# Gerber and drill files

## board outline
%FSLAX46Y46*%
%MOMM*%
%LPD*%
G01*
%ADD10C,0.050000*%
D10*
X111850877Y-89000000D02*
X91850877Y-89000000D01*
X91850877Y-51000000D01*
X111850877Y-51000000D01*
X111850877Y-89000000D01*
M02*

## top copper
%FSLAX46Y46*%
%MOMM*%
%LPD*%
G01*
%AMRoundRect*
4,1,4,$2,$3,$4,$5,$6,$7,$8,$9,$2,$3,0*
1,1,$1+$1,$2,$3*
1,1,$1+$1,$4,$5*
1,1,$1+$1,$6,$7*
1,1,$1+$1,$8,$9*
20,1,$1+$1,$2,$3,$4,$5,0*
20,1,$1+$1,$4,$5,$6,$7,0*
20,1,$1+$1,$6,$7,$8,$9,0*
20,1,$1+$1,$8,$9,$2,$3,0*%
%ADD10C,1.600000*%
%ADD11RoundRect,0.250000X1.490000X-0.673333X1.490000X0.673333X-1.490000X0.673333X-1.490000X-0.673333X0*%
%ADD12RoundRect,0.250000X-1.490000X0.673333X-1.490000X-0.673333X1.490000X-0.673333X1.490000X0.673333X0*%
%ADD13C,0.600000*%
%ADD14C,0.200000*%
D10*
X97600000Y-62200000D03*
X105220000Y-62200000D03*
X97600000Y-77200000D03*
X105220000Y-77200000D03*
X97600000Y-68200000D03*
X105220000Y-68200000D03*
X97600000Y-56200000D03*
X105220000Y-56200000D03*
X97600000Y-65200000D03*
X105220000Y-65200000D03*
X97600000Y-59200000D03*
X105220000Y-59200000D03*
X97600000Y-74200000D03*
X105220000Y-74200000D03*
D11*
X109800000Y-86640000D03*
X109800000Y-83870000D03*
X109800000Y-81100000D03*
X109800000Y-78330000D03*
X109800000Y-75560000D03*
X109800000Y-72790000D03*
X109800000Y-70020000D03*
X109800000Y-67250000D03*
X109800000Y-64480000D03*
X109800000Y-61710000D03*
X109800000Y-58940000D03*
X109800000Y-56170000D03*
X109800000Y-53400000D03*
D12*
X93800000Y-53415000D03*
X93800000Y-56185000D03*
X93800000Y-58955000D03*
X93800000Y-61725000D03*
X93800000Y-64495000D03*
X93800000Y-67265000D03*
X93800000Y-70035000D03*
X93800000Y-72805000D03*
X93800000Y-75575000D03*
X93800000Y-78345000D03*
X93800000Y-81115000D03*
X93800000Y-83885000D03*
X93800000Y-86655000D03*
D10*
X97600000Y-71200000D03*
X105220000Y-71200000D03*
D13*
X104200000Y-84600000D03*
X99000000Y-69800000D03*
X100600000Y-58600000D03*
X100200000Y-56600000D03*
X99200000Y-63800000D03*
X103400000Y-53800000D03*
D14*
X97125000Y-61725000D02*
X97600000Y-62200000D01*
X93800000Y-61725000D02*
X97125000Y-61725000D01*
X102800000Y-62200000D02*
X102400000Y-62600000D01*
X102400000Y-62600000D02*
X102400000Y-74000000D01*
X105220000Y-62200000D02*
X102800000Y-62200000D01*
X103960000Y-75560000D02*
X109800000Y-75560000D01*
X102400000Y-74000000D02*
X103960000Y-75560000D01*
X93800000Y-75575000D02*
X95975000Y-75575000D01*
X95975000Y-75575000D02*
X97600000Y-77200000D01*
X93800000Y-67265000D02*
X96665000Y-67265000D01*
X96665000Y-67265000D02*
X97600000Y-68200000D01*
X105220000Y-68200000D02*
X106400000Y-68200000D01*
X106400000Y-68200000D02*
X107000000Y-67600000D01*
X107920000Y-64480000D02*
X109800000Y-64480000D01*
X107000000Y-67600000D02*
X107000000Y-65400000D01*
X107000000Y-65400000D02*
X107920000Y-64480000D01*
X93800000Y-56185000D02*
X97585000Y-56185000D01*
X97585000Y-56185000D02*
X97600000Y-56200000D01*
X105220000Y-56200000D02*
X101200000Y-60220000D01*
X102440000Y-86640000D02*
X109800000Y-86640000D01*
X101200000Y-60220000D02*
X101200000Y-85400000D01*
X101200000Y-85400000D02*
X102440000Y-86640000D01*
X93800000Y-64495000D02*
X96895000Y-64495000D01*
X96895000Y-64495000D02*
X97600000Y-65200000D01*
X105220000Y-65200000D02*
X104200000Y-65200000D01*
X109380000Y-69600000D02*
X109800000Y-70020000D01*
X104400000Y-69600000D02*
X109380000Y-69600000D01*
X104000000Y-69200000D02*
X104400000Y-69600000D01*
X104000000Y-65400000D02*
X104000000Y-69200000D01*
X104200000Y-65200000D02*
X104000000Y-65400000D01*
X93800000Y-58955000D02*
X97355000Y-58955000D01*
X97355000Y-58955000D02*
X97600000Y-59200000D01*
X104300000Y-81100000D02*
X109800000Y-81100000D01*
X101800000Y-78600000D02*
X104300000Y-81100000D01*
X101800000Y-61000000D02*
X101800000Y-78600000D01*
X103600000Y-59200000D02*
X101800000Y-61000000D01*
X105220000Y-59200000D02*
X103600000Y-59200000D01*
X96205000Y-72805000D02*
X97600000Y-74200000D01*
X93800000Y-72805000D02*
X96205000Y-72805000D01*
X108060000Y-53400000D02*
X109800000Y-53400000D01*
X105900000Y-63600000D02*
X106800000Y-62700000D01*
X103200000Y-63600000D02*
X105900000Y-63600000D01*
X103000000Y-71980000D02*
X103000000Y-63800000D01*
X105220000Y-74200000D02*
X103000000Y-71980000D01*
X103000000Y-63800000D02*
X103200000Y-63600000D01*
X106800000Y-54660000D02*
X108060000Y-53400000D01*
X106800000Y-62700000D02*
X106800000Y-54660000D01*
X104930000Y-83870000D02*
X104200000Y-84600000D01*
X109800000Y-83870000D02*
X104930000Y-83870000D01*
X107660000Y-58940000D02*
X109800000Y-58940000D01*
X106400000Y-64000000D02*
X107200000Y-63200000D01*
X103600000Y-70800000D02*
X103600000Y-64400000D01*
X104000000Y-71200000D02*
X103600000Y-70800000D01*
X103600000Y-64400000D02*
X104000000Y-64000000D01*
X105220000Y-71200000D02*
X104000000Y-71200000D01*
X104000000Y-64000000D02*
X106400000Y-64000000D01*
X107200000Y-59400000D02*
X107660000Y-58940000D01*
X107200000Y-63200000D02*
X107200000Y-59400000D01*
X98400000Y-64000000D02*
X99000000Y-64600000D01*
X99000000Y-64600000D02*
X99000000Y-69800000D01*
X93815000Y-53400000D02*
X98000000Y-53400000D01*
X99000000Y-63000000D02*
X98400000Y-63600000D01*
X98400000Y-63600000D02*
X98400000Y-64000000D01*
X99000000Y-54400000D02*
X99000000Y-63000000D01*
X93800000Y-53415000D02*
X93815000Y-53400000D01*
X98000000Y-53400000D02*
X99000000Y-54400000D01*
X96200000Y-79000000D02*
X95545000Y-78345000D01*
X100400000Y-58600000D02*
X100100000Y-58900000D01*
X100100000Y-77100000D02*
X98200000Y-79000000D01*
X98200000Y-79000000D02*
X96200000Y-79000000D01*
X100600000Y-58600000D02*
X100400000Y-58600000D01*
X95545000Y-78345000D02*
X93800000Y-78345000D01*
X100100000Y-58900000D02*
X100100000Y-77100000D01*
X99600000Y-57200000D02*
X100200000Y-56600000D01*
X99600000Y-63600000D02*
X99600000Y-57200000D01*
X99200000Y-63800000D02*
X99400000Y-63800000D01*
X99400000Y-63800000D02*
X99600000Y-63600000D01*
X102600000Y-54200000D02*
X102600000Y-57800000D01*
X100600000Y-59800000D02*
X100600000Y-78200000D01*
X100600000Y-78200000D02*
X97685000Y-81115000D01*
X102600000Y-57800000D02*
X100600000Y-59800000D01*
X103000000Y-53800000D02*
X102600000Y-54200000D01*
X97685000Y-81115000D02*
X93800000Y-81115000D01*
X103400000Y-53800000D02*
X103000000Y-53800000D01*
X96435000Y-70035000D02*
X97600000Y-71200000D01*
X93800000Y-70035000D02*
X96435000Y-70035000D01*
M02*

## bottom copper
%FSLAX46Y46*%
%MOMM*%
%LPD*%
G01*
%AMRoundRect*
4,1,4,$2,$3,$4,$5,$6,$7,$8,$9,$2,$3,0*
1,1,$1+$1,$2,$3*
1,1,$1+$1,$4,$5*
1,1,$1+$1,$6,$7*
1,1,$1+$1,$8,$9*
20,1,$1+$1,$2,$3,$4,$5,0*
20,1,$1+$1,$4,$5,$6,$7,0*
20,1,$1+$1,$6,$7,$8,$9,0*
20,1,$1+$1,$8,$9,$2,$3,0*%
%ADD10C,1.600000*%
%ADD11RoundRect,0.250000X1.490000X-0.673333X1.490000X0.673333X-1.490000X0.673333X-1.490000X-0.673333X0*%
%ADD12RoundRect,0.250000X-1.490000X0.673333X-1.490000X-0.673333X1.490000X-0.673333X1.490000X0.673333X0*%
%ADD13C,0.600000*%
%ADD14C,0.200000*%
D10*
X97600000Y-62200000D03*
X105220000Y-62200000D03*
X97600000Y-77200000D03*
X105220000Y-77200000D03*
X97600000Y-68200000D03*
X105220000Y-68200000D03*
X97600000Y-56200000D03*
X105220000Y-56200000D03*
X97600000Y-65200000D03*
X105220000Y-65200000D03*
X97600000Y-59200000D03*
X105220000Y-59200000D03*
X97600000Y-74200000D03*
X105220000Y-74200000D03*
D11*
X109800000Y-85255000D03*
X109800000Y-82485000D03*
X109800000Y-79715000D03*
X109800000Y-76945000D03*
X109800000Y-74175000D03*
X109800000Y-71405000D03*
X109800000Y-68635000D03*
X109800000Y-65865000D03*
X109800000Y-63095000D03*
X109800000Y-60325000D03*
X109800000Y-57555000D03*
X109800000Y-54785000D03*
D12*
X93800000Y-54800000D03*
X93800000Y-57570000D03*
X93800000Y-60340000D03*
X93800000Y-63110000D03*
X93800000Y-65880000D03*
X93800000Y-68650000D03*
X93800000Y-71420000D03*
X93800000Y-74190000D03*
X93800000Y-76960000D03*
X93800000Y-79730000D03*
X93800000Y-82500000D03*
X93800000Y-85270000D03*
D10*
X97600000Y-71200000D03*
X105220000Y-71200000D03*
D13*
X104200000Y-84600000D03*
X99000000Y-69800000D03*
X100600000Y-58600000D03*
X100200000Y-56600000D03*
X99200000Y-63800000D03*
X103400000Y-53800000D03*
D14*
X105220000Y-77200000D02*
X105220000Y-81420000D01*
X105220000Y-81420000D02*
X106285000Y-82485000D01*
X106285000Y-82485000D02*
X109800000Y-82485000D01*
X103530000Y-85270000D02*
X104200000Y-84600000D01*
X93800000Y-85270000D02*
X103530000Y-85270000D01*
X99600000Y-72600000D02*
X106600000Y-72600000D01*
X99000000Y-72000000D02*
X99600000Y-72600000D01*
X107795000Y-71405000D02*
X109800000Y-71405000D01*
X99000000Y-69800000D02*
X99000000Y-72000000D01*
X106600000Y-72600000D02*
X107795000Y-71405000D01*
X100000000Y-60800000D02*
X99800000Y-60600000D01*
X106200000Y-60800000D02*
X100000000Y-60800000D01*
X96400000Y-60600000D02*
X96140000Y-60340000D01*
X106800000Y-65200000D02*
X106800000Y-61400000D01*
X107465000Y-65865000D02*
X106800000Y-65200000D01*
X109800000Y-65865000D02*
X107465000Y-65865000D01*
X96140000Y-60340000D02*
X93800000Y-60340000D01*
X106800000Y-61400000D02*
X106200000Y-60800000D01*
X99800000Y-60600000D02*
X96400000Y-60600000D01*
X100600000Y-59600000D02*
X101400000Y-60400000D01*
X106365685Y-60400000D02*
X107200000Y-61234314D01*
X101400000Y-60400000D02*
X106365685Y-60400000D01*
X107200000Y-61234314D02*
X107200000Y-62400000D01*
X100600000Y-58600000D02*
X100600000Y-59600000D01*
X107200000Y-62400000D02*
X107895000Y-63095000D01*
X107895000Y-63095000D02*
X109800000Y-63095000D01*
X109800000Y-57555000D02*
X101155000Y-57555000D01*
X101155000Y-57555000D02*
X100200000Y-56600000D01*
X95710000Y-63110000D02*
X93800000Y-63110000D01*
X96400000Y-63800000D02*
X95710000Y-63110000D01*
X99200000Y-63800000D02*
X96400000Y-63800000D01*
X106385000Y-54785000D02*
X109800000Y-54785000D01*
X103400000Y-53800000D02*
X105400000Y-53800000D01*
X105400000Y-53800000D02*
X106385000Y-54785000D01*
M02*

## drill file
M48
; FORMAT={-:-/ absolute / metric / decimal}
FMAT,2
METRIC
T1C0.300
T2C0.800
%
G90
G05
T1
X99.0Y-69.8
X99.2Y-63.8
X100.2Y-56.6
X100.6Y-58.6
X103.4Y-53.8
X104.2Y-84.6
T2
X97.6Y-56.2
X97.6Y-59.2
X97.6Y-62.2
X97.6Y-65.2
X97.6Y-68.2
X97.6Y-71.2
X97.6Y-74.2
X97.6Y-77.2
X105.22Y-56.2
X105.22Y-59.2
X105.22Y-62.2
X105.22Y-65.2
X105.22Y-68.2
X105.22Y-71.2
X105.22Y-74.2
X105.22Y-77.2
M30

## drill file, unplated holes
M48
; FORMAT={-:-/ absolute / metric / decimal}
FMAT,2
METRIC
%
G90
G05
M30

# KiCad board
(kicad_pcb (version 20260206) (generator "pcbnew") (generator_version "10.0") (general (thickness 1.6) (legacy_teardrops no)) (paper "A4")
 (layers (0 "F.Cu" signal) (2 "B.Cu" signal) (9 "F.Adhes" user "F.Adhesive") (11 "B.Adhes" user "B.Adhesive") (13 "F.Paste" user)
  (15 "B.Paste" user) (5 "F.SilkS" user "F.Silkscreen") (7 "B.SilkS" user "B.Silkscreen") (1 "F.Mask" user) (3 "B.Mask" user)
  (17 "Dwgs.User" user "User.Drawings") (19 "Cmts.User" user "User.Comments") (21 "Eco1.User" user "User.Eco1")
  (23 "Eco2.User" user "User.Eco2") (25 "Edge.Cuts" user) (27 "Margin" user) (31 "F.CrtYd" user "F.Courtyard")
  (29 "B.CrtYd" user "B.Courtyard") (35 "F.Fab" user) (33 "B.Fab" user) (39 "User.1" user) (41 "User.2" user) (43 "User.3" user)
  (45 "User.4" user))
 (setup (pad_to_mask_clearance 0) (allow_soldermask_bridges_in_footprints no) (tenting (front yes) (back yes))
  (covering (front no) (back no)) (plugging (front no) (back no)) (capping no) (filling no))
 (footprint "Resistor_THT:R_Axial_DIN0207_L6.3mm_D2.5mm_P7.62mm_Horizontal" (layer "F.Cu") (at 97.6 62.2)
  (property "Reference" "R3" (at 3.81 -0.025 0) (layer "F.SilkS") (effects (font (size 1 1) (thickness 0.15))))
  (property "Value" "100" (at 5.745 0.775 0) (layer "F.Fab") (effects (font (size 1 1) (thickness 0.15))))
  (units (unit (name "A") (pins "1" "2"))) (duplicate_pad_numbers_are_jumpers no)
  (pad "1" thru_hole circle (at 0 0) (size 1.6 1.6) (drill 0.8) (layers "*.Cu" "*.Mask") (remove_unused_layers no) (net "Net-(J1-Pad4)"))
  (pad "2" thru_hole circle (at 7.62 0) (size 1.6 1.6) (drill 0.8) (layers "*.Cu" "*.Mask") (remove_unused_layers no) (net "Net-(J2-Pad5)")))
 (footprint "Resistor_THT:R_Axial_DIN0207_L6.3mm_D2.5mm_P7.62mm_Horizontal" (layer "F.Cu") (at 97.6 77.2)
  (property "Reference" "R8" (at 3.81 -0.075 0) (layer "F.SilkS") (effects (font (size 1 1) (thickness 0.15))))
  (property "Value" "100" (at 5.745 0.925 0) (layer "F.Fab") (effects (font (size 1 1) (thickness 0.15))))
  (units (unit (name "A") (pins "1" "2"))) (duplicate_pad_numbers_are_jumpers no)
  (pad "1" thru_hole circle (at 0 0) (size 1.6 1.6) (drill 0.8) (layers "*.Cu" "*.Mask") (remove_unused_layers no) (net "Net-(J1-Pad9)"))
  (pad "2" thru_hole circle (at 7.62 0) (size 1.6 1.6) (drill 0.8) (layers "*.Cu" "*.Mask") (remove_unused_layers no) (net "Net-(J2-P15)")))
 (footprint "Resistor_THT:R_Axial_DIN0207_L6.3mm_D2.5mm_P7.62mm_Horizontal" (layer "F.Cu") (at 97.6 68.2)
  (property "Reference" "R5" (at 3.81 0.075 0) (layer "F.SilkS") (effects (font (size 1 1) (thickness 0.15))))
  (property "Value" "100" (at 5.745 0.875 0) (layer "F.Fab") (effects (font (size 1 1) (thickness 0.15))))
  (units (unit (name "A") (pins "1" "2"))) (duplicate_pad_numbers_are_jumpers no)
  (pad "1" thru_hole circle (at 0 0) (size 1.6 1.6) (drill 0.8) (layers "*.Cu" "*.Mask") (remove_unused_layers no) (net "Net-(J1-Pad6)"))
  (pad "2" thru_hole circle (at 7.62 0) (size 1.6 1.6) (drill 0.8) (layers "*.Cu" "*.Mask") (remove_unused_layers no) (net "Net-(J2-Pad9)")))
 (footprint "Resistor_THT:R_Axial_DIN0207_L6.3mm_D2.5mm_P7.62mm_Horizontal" (layer "F.Cu") (at 97.6 56.2)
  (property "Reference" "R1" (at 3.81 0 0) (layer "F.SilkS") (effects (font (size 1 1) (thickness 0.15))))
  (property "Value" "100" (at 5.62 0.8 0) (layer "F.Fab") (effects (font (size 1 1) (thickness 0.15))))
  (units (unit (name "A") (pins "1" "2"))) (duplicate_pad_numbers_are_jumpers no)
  (pad "1" thru_hole circle (at 0 0) (size 1.6 1.6) (drill 0.8) (layers "*.Cu" "*.Mask") (remove_unused_layers no) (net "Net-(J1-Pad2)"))
  (pad "2" thru_hole circle (at 7.62 0) (size 1.6 1.6) (drill 0.8) (layers "*.Cu" "*.Mask") (remove_unused_layers no) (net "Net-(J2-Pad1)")))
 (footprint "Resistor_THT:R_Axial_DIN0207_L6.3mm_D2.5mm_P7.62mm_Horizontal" (layer "F.Cu") (at 97.6 65.2)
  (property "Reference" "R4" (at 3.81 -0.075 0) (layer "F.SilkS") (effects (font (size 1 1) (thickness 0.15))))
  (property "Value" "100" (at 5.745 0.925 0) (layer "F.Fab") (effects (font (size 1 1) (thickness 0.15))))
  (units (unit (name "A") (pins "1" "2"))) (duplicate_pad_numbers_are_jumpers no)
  (pad "1" thru_hole circle (at 0 0) (size 1.6 1.6) (drill 0.8) (layers "*.Cu" "*.Mask") (remove_unused_layers no) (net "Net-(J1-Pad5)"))
  (pad "2" thru_hole circle (at 7.62 0) (size 1.6 1.6) (drill 0.8) (layers "*.Cu" "*.Mask") (remove_unused_layers no) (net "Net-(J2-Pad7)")))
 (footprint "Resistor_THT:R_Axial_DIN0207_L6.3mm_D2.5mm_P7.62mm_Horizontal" (layer "F.Cu") (at 97.6 59.2)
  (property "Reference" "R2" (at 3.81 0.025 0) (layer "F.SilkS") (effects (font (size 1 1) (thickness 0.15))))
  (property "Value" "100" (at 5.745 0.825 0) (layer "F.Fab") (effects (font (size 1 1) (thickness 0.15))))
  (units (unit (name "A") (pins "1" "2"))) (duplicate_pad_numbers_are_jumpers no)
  (pad "1" thru_hole circle (at 0 0) (size 1.6 1.6) (drill 0.8) (layers "*.Cu" "*.Mask") (remove_unused_layers no) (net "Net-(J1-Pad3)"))
  (pad "2" thru_hole circle (at 7.62 0) (size 1.6 1.6) (drill 0.8) (layers "*.Cu" "*.Mask") (remove_unused_layers no) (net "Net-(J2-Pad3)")))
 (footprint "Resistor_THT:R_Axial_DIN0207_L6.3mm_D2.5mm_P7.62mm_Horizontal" (layer "F.Cu") (at 97.6 74.2)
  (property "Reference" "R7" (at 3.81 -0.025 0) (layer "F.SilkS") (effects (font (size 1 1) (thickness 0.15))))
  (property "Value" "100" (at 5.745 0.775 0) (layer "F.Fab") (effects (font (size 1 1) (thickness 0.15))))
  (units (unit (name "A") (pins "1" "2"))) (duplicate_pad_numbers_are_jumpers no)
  (pad "1" thru_hole circle (at 0 0) (size 1.6 1.6) (drill 0.8) (layers "*.Cu" "*.Mask") (remove_unused_layers no) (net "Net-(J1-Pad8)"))
  (pad "2" thru_hole circle (at 7.62 0) (size 1.6 1.6) (drill 0.8) (layers "*.Cu" "*.Mask") (remove_unused_layers no) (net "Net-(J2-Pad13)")))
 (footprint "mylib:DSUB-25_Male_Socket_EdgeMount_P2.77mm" (layer "F.Cu") (at 116.84 77.06 180)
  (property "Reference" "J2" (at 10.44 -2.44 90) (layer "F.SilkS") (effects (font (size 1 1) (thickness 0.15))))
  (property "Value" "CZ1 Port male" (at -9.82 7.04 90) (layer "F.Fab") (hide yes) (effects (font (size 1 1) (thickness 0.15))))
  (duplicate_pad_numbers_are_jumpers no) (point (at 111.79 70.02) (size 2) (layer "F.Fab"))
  (pad "1" smd roundrect (at 7.04 -9.58 90) (size 1.846667 3.48) (layers "F.Cu" "F.Mask" "F.Paste") (roundrect_rratio 0.135379)
   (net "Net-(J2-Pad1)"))
  (pad "2" smd roundrect (at 7.04 -6.81 90) (size 1.846667 3.48) (layers "F.Cu" "F.Mask" "F.Paste") (roundrect_rratio 0.135379) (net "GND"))
  (pad "3" smd roundrect (at 7.04 -4.04 90) (size 1.846667 3.48) (layers "F.Cu" "F.Mask" "F.Paste") (roundrect_rratio 0.135379)
   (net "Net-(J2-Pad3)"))
  (pad "4" smd roundrect (at 7.04 -1.27 90) (size 1.846667 3.48) (layers "F.Cu" "F.Mask" "F.Paste") (roundrect_rratio 0.135379)
   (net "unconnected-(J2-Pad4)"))
  (pad "5" smd roundrect (at 7.04 1.5 90) (size 1.846667 3.48) (layers "F.Cu" "F.Mask" "F.Paste") (roundrect_rratio 0.135379)
   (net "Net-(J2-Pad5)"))
  (pad "6" smd roundrect (at 7.04 4.27 90) (size 1.846667 3.48) (layers "F.Cu" "F.Mask" "F.Paste") (roundrect_rratio 0.135379)
   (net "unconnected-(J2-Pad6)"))
  (pad "7" smd roundrect (at 7.04 7.04 90) (size 1.846667 3.48) (layers "F.Cu" "F.Mask" "F.Paste") (roundrect_rratio 0.135379)
   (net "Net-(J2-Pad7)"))
  (pad "8" smd roundrect (at 7.04 9.81 90) (size 1.846667 3.48) (layers "F.Cu" "F.Mask" "F.Paste") (roundrect_rratio 0.135379)
   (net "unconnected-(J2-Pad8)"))
  (pad "9" smd roundrect (at 7.04 12.58 90) (size 1.846667 3.48) (layers "F.Cu" "F.Mask" "F.Paste") (roundrect_rratio 0.135379)
   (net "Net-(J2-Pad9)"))
  (pad "10" smd roundrect (at 7.04 15.35 90) (size 1.846667 3.48) (layers "F.Cu" "F.Mask" "F.Paste") (roundrect_rratio 0.135379)
   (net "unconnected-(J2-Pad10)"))
  (pad "11" smd roundrect (at 7.04 18.12 90) (size 1.846667 3.48) (layers "F.Cu" "F.Mask" "F.Paste") (roundrect_rratio 0.135379)
   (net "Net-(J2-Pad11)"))
  (pad "12" smd roundrect (at 7.04 20.89 90) (size 1.846667 3.48) (layers "F.Cu" "F.Mask" "F.Paste") (roundrect_rratio 0.135379)
   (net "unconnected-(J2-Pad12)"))
  (pad "13" smd roundrect (at 7.04 23.66 90) (size 1.846667 3.48) (layers "F.Cu" "F.Mask" "F.Paste") (roundrect_rratio 0.135379)
   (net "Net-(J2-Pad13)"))
  (pad "14" smd roundrect (at 7.04 -8.195 90) (size 1.846667 3.48) (layers "B.Cu" "B.Mask" "B.Paste") (roundrect_rratio 0.135379)
   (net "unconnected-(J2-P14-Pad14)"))
  (pad "15" smd roundrect (at 7.04 -5.425 90) (size 1.846667 3.48) (layers "B.Cu" "B.Mask" "B.Paste") (roundrect_rratio 0.135379)
   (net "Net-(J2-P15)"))
  (pad "16" smd roundrect (at 7.04 -2.655 90) (size 1.846667 3.48) (layers "B.Cu" "B.Mask" "B.Paste") (roundrect_rratio 0.135379)
   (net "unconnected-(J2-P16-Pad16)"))
  (pad "17" smd roundrect (at 7.04 0.115 90) (size 1.846667 3.48) (layers "B.Cu" "B.Mask" "B.Paste") (roundrect_rratio 0.135379)
   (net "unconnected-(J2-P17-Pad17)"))
  (pad "18" smd roundrect (at 7.04 2.885 90) (size 1.846667 3.48) (layers "B.Cu" "B.Mask" "B.Paste") (roundrect_rratio 0.135379)
   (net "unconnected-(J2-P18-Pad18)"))
  (pad "19" smd roundrect (at 7.04 5.655 90) (size 1.846667 3.48) (layers "B.Cu" "B.Mask" "B.Paste") (roundrect_rratio 0.135379)
   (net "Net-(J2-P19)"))
  (pad "20" smd roundrect (at 7.04 8.425 90) (size 1.846667 3.48) (layers "B.Cu" "B.Mask" "B.Paste") (roundrect_rratio 0.135379)
   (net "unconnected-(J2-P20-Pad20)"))
  (pad "21" smd roundrect (at 7.04 11.195 90) (size 1.846667 3.48) (layers "B.Cu" "B.Mask" "B.Paste") (roundrect_rratio 0.135379)
   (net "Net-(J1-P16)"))
  (pad "22" smd roundrect (at 7.04 13.965 90) (size 1.846667 3.48) (layers "B.Cu" "B.Mask" "B.Paste") (roundrect_rratio 0.135379)
   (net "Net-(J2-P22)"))
  (pad "23" smd roundrect (at 7.04 16.735 90) (size 1.846667 3.48) (layers "B.Cu" "B.Mask" "B.Paste") (roundrect_rratio 0.135379)
   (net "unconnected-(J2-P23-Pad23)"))
  (pad "24" smd roundrect (at 7.04 19.505 90) (size 1.846667 3.48) (layers "B.Cu" "B.Mask" "B.Paste") (roundrect_rratio 0.135379)
   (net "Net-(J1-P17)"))
  (pad "25" smd roundrect (at 7.04 22.275 90) (size 1.846667 3.48) (layers "B.Cu" "B.Mask" "B.Paste") (roundrect_rratio 0.135379)
   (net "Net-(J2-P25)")))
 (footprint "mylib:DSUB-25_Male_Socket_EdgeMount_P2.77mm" (layer "F.Cu") (at 86.76 62.995)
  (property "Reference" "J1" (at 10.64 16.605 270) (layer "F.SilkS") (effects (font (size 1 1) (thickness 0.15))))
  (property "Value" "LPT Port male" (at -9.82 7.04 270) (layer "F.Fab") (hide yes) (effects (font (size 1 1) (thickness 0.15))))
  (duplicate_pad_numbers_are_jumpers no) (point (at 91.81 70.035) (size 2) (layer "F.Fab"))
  (pad "1" smd roundrect (at 7.04 -9.58 270) (size 1.846667 3.48) (layers "F.Cu" "F.Mask" "F.Paste") (roundrect_rratio 0.135379)
   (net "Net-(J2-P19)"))
  (pad "2" smd roundrect (at 7.04 -6.81 270) (size 1.846667 3.48) (layers "F.Cu" "F.Mask" "F.Paste") (roundrect_rratio 0.135379)
   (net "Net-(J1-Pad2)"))
  (pad "3" smd roundrect (at 7.04 -4.04 270) (size 1.846667 3.48) (layers "F.Cu" "F.Mask" "F.Paste") (roundrect_rratio 0.135379)
   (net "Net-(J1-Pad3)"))
  (pad "4" smd roundrect (at 7.04 -1.27 270) (size 1.846667 3.48) (layers "F.Cu" "F.Mask" "F.Paste") (roundrect_rratio 0.135379)
   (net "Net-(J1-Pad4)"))
  (pad "5" smd roundrect (at 7.04 1.5 270) (size 1.846667 3.48) (layers "F.Cu" "F.Mask" "F.Paste") (roundrect_rratio 0.135379)
   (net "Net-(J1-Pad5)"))
  (pad "6" smd roundrect (at 7.04 4.27 270) (size 1.846667 3.48) (layers "F.Cu" "F.Mask" "F.Paste") (roundrect_rratio 0.135379)
   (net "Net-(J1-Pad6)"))
  (pad "7" smd roundrect (at 7.04 7.04 270) (size 1.846667 3.48) (layers "F.Cu" "F.Mask" "F.Paste") (roundrect_rratio 0.135379)
   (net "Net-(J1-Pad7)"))
  (pad "8" smd roundrect (at 7.04 9.81 270) (size 1.846667 3.48) (layers "F.Cu" "F.Mask" "F.Paste") (roundrect_rratio 0.135379)
   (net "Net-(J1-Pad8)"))
  (pad "9" smd roundrect (at 7.04 12.58 270) (size 1.846667 3.48) (layers "F.Cu" "F.Mask" "F.Paste") (roundrect_rratio 0.135379)
   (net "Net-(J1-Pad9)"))
  (pad "10" smd roundrect (at 7.04 15.35 270) (size 1.846667 3.48) (layers "F.Cu" "F.Mask" "F.Paste") (roundrect_rratio 0.135379)
   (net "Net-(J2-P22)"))
  (pad "11" smd roundrect (at 7.04 18.12 270) (size 1.846667 3.48) (layers "F.Cu" "F.Mask" "F.Paste") (roundrect_rratio 0.135379)
   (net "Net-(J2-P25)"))
  (pad "12" smd roundrect (at 7.04 20.89 270) (size 1.846667 3.48) (layers "F.Cu" "F.Mask" "F.Paste") (roundrect_rratio 0.135379)
   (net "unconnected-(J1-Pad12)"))
  (pad "13" smd roundrect (at 7.04 23.66 270) (size 1.846667 3.48) (layers "F.Cu" "F.Mask" "F.Paste") (roundrect_rratio 0.135379)
   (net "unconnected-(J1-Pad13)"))
  (pad "14" smd roundrect (at 7.04 -8.195 270) (size 1.846667 3.48) (layers "B.Cu" "B.Mask" "B.Paste") (roundrect_rratio 0.135379)
   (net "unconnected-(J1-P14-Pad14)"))
  (pad "15" smd roundrect (at 7.04 -5.425 270) (size 1.846667 3.48) (layers "B.Cu" "B.Mask" "B.Paste") (roundrect_rratio 0.135379)
   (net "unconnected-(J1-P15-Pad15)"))
  (pad "16" smd roundrect (at 7.04 -2.655 270) (size 1.846667 3.48) (layers "B.Cu" "B.Mask" "B.Paste") (roundrect_rratio 0.135379)
   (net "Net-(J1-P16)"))
  (pad "17" smd roundrect (at 7.04 0.115 270) (size 1.846667 3.48) (layers "B.Cu" "B.Mask" "B.Paste") (roundrect_rratio 0.135379)
   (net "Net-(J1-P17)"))
  (pad "18" smd roundrect (at 7.04 2.885 270) (size 1.846667 3.48) (layers "B.Cu" "B.Mask" "B.Paste") (roundrect_rratio 0.135379)
   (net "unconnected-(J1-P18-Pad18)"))
  (pad "19" smd roundrect (at 7.04 5.655 270) (size 1.846667 3.48) (layers "B.Cu" "B.Mask" "B.Paste") (roundrect_rratio 0.135379)
   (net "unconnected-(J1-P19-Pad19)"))
  (pad "20" smd roundrect (at 7.04 8.425 270) (size 1.846667 3.48) (layers "B.Cu" "B.Mask" "B.Paste") (roundrect_rratio 0.135379)
   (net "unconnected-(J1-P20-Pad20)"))
  (pad "21" smd roundrect (at 7.04 11.195 270) (size 1.846667 3.48) (layers "B.Cu" "B.Mask" "B.Paste") (roundrect_rratio 0.135379)
   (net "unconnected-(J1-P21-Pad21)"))
  (pad "22" smd roundrect (at 7.04 13.965 270) (size 1.846667 3.48) (layers "B.Cu" "B.Mask" "B.Paste") (roundrect_rratio 0.135379)
   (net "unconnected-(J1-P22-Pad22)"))
  (pad "23" smd roundrect (at 7.04 16.735 270) (size 1.846667 3.48) (layers "B.Cu" "B.Mask" "B.Paste") (roundrect_rratio 0.135379)
   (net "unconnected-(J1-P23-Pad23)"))
  (pad "24" smd roundrect (at 7.04 19.505 270) (size 1.846667 3.48) (layers "B.Cu" "B.Mask" "B.Paste") (roundrect_rratio 0.135379)
   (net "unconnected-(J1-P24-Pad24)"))
  (pad "25" smd roundrect (at 7.04 22.275 270) (size 1.846667 3.48) (layers "B.Cu" "B.Mask" "B.Paste") (roundrect_rratio 0.135379)
   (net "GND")))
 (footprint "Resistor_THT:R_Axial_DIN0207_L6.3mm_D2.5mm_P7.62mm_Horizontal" (layer "F.Cu") (at 97.6 71.2)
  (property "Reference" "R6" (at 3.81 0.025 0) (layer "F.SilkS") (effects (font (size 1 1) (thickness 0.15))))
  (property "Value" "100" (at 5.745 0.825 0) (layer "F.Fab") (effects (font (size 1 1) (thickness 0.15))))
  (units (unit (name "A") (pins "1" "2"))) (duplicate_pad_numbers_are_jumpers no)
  (pad "1" thru_hole circle (at 0 0) (size 1.6 1.6) (drill 0.8) (layers "*.Cu" "*.Mask") (remove_unused_layers no) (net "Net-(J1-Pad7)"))
  (pad "2" thru_hole circle (at 7.62 0) (size 1.6 1.6) (drill 0.8) (layers "*.Cu" "*.Mask") (remove_unused_layers no) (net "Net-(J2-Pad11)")))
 (gr_poly
  (pts (xy 91.850877 51) (xy 91.850877 89) (xy 111.850877 89) (xy 111.850877 51)) (stroke (width 0.05) (type solid)) (fill no)
  (layer "Edge.Cuts"))
 (segment (start 97.125 61.725) (end 97.6 62.2) (width 0.2) (layer "F.Cu") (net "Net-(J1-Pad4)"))
 (segment (start 93.8 61.725) (end 97.125 61.725) (width 0.2) (layer "F.Cu") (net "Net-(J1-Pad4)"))
 (segment (start 102.8 62.2) (end 102.4 62.6) (width 0.2) (layer "F.Cu") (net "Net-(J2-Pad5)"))
 (segment (start 102.4 62.6) (end 102.4 74) (width 0.2) (layer "F.Cu") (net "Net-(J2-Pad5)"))
 (segment (start 105.22 62.2) (end 102.8 62.2) (width 0.2) (layer "F.Cu") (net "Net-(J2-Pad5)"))
 (segment (start 103.96 75.56) (end 109.8 75.56) (width 0.2) (layer "F.Cu") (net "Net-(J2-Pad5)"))
 (segment (start 102.4 74) (end 103.96 75.56) (width 0.2) (layer "F.Cu") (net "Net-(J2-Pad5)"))
 (segment (start 93.8 75.575) (end 95.975 75.575) (width 0.2) (layer "F.Cu") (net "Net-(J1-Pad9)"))
 (segment (start 95.975 75.575) (end 97.6 77.2) (width 0.2) (layer "F.Cu") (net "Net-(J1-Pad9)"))
 (segment (start 105.22 77.2) (end 105.22 81.42) (width 0.2) (layer "B.Cu") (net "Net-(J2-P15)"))
 (segment (start 105.22 81.42) (end 106.285 82.485) (width 0.2) (layer "B.Cu") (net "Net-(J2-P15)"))
 (segment (start 106.285 82.485) (end 109.8 82.485) (width 0.2) (layer "B.Cu") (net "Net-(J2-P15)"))
 (segment (start 93.8 67.265) (end 96.665 67.265) (width 0.2) (layer "F.Cu") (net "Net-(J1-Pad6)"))
 (segment (start 96.665 67.265) (end 97.6 68.2) (width 0.2) (layer "F.Cu") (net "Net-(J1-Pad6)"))
 (segment (start 105.22 68.2) (end 106.4 68.2) (width 0.2) (layer "F.Cu") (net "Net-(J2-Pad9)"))
 (segment (start 106.4 68.2) (end 107 67.6) (width 0.2) (layer "F.Cu") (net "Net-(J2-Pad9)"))
 (segment (start 107.92 64.48) (end 109.8 64.48) (width 0.2) (layer "F.Cu") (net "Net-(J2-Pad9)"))
 (segment (start 107 67.6) (end 107 65.4) (width 0.2) (layer "F.Cu") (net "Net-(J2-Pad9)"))
 (segment (start 107 65.4) (end 107.92 64.48) (width 0.2) (layer "F.Cu") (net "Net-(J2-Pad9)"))
 (segment (start 93.8 56.185) (end 97.585 56.185) (width 0.2) (layer "F.Cu") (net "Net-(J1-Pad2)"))
 (segment (start 97.585 56.185) (end 97.6 56.2) (width 0.2) (layer "F.Cu") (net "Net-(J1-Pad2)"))
 (segment (start 105.22 56.2) (end 101.2 60.22) (width 0.2) (layer "F.Cu") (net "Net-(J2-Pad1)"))
 (segment (start 102.44 86.64) (end 109.8 86.64) (width 0.2) (layer "F.Cu") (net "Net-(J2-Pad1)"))
 (segment (start 101.2 60.22) (end 101.2 85.4) (width 0.2) (layer "F.Cu") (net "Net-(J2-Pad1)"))
 (segment (start 101.2 85.4) (end 102.44 86.64) (width 0.2) (layer "F.Cu") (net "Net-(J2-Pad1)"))
 (segment (start 93.8 64.495) (end 96.895 64.495) (width 0.2) (layer "F.Cu") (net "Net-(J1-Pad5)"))
 (segment (start 96.895 64.495) (end 97.6 65.2) (width 0.2) (layer "F.Cu") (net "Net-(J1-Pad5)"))
 (segment (start 105.22 65.2) (end 104.2 65.2) (width 0.2) (layer "F.Cu") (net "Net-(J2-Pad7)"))
 (segment (start 109.38 69.6) (end 109.8 70.02) (width 0.2) (layer "F.Cu") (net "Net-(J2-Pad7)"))
 (segment (start 104.4 69.6) (end 109.38 69.6) (width 0.2) (layer "F.Cu") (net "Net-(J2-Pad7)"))
 (segment (start 104 69.2) (end 104.4 69.6) (width 0.2) (layer "F.Cu") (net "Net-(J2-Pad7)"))
 (segment (start 104 65.4) (end 104 69.2) (width 0.2) (layer "F.Cu") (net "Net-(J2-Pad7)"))
 (segment (start 104.2 65.2) (end 104 65.4) (width 0.2) (layer "F.Cu") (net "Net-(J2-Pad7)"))
 (segment (start 93.8 58.955) (end 97.355 58.955) (width 0.2) (layer "F.Cu") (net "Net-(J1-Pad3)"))
 (segment (start 97.355 58.955) (end 97.6 59.2) (width 0.2) (layer "F.Cu") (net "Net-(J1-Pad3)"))
 (segment (start 104.3 81.1) (end 109.8 81.1) (width 0.2) (layer "F.Cu") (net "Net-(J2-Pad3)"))
 (segment (start 101.8 78.6) (end 104.3 81.1) (width 0.2) (layer "F.Cu") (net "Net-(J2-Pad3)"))
 (segment (start 101.8 61) (end 101.8 78.6) (width 0.2) (layer "F.Cu") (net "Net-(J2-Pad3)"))
 (segment (start 103.6 59.2) (end 101.8 61) (width 0.2) (layer "F.Cu") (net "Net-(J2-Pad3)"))
 (segment (start 105.22 59.2) (end 103.6 59.2) (width 0.2) (layer "F.Cu") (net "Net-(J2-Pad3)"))
 (segment (start 96.205 72.805) (end 97.6 74.2) (width 0.2) (layer "F.Cu") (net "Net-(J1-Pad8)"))
 (segment (start 93.8 72.805) (end 96.205 72.805) (width 0.2) (layer "F.Cu") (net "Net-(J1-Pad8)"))
 (segment (start 108.06 53.4) (end 109.8 53.4) (width 0.2) (layer "F.Cu") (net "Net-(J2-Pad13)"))
 (segment (start 105.9 63.6) (end 106.8 62.7) (width 0.2) (layer "F.Cu") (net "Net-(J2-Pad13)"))
 (segment (start 103.2 63.6) (end 105.9 63.6) (width 0.2) (layer "F.Cu") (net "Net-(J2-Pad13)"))
 (segment (start 103 71.98) (end 103 63.8) (width 0.2) (layer "F.Cu") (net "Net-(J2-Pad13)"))
 (segment (start 105.22 74.2) (end 103 71.98) (width 0.2) (layer "F.Cu") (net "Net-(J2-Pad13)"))
 (segment (start 103 63.8) (end 103.2 63.6) (width 0.2) (layer "F.Cu") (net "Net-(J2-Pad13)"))
 (segment (start 106.8 54.66) (end 108.06 53.4) (width 0.2) (layer "F.Cu") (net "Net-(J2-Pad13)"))
 (segment (start 106.8 62.7) (end 106.8 54.66) (width 0.2) (layer "F.Cu") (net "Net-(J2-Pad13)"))
 (segment (start 104.93 83.87) (end 104.2 84.6) (width 0.2) (layer "F.Cu") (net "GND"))
 (segment (start 109.8 83.87) (end 104.93 83.87) (width 0.2) (layer "F.Cu") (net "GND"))
 (via (at 104.2 84.6) (size 0.6) (drill 0.3) (layers "F.Cu" "B.Cu") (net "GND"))
 (segment (start 103.53 85.27) (end 104.2 84.6) (width 0.2) (layer "B.Cu") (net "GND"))
 (segment (start 93.8 85.27) (end 103.53 85.27) (width 0.2) (layer "B.Cu") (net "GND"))
 (segment (start 107.66 58.94) (end 109.8 58.94) (width 0.2) (layer "F.Cu") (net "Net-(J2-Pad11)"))
 (segment (start 106.4 64) (end 107.2 63.2) (width 0.2) (layer "F.Cu") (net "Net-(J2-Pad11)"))
 (segment (start 103.6 70.8) (end 103.6 64.4) (width 0.2) (layer "F.Cu") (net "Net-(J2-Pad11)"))
 (segment (start 104 71.2) (end 103.6 70.8) (width 0.2) (layer "F.Cu") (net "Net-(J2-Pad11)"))
 (segment (start 103.6 64.4) (end 104 64) (width 0.2) (layer "F.Cu") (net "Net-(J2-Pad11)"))
 (segment (start 105.22 71.2) (end 104 71.2) (width 0.2) (layer "F.Cu") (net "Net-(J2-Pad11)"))
 (segment (start 104 64) (end 106.4 64) (width 0.2) (layer "F.Cu") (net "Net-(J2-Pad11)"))
 (segment (start 107.2 59.4) (end 107.66 58.94) (width 0.2) (layer "F.Cu") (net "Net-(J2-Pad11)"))
 (segment (start 107.2 63.2) (end 107.2 59.4) (width 0.2) (layer "F.Cu") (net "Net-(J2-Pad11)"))
 (segment (start 98.4 64) (end 99 64.6) (width 0.2) (layer "F.Cu") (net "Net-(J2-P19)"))
 (segment (start 99 64.6) (end 99 69.8) (width 0.2) (layer "F.Cu") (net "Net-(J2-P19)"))
 (segment (start 93.815 53.4) (end 98 53.4) (width 0.2) (layer "F.Cu") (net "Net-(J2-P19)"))
 (segment (start 99 63) (end 98.4 63.6) (width 0.2) (layer "F.Cu") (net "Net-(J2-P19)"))
 (segment (start 98.4 63.6) (end 98.4 64) (width 0.2) (layer "F.Cu") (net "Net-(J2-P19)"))
 (segment (start 99 54.4) (end 99 63) (width 0.2) (layer "F.Cu") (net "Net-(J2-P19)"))
 (segment (start 93.8 53.415) (end 93.815 53.4) (width 0.2) (layer "F.Cu") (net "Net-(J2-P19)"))
 (segment (start 98 53.4) (end 99 54.4) (width 0.2) (layer "F.Cu") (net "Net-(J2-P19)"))
 (via (at 99 69.8) (size 0.6) (drill 0.3) (layers "F.Cu" "B.Cu") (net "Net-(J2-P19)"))
 (segment (start 99.6 72.6) (end 106.6 72.6) (width 0.2) (layer "B.Cu") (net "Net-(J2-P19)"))
 (segment (start 99 72) (end 99.6 72.6) (width 0.2) (layer "B.Cu") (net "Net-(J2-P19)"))
 (segment (start 107.795 71.405) (end 109.8 71.405) (width 0.2) (layer "B.Cu") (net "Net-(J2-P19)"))
 (segment (start 99 69.8) (end 99 72) (width 0.2) (layer "B.Cu") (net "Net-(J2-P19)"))
 (segment (start 106.6 72.6) (end 107.795 71.405) (width 0.2) (layer "B.Cu") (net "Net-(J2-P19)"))
 (segment (start 100 60.8) (end 99.8 60.6) (width 0.2) (layer "B.Cu") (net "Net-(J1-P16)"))
 (segment (start 106.2 60.8) (end 100 60.8) (width 0.2) (layer "B.Cu") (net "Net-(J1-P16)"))
 (segment (start 96.4 60.6) (end 96.14 60.34) (width 0.2) (layer "B.Cu") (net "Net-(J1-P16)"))
 (segment (start 106.8 65.2) (end 106.8 61.4) (width 0.2) (layer "B.Cu") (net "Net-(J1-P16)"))
 (segment (start 107.465 65.865) (end 106.8 65.2) (width 0.2) (layer "B.Cu") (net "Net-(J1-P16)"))
 (segment (start 109.8 65.865) (end 107.465 65.865) (width 0.2) (layer "B.Cu") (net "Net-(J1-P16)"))
 (segment (start 96.14 60.34) (end 93.8 60.34) (width 0.2) (layer "B.Cu") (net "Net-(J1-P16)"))
 (segment (start 106.8 61.4) (end 106.2 60.8) (width 0.2) (layer "B.Cu") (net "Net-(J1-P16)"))
 (segment (start 99.8 60.6) (end 96.4 60.6) (width 0.2) (layer "B.Cu") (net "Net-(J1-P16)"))
 (segment (start 96.2 79) (end 95.545 78.345) (width 0.2) (layer "F.Cu") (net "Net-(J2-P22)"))
 (segment (start 100.4 58.6) (end 100.1 58.9) (width 0.2) (layer "F.Cu") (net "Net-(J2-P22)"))
 (segment (start 100.1 77.1) (end 98.2 79) (width 0.2) (layer "F.Cu") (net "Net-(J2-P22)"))
 (segment (start 98.2 79) (end 96.2 79) (width 0.2) (layer "F.Cu") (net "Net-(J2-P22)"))
 (segment (start 100.6 58.6) (end 100.4 58.6) (width 0.2) (layer "F.Cu") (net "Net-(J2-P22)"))
 (segment (start 95.545 78.345) (end 93.8 78.345) (width 0.2) (layer "F.Cu") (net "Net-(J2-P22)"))
 (segment (start 100.1 58.9) (end 100.1 77.1) (width 0.2) (layer "F.Cu") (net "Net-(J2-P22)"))
 (via (at 100.6 58.6) (size 0.6) (drill 0.3) (layers "F.Cu" "B.Cu") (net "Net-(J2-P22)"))
 (segment (start 100.6 59.6) (end 101.4 60.4) (width 0.2) (layer "B.Cu") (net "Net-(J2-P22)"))
 (segment (start 106.365685 60.4) (end 107.2 61.234314) (width 0.2) (layer "B.Cu") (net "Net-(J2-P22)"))
 (segment (start 101.4 60.4) (end 106.365685 60.4) (width 0.2) (layer "B.Cu") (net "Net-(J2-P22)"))
 (segment (start 107.2 61.234314) (end 107.2 62.4) (width 0.2) (layer "B.Cu") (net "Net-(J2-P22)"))
 (segment (start 100.6 58.6) (end 100.6 59.6) (width 0.2) (layer "B.Cu") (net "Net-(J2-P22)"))
 (segment (start 107.2 62.4) (end 107.895 63.095) (width 0.2) (layer "B.Cu") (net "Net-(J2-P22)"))
 (segment (start 107.895 63.095) (end 109.8 63.095) (width 0.2) (layer "B.Cu") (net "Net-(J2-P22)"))
 (segment (start 99.6 57.2) (end 100.2 56.6) (width 0.2) (layer "F.Cu") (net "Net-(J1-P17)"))
 (segment (start 99.6 63.6) (end 99.6 57.2) (width 0.2) (layer "F.Cu") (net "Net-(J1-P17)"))
 (segment (start 99.2 63.8) (end 99.4 63.8) (width 0.2) (layer "F.Cu") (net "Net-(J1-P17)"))
 (segment (start 99.4 63.8) (end 99.6 63.6) (width 0.2) (layer "F.Cu") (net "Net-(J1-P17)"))
 (via (at 100.2 56.6) (size 0.6) (drill 0.3) (layers "F.Cu" "B.Cu") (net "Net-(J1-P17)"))
 (via (at 99.2 63.8) (size 0.6) (drill 0.3) (layers "F.Cu" "B.Cu") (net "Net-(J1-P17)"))
 (segment (start 109.8 57.555) (end 101.155 57.555) (width 0.2) (layer "B.Cu") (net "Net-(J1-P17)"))
 (segment (start 101.155 57.555) (end 100.2 56.6) (width 0.2) (layer "B.Cu") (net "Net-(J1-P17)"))
 (segment (start 95.71 63.11) (end 93.8 63.11) (width 0.2) (layer "B.Cu") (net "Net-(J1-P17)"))
 (segment (start 96.4 63.8) (end 95.71 63.11) (width 0.2) (layer "B.Cu") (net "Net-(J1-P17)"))
 (segment (start 99.2 63.8) (end 96.4 63.8) (width 0.2) (layer "B.Cu") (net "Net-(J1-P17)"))
 (segment (start 102.6 54.2) (end 102.6 57.8) (width 0.2) (layer "F.Cu") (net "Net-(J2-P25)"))
 (segment (start 100.6 59.8) (end 100.6 78.2) (width 0.2) (layer "F.Cu") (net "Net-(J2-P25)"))
 (segment (start 100.6 78.2) (end 97.685 81.115) (width 0.2) (layer "F.Cu") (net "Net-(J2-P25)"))
 (segment (start 102.6 57.8) (end 100.6 59.8) (width 0.2) (layer "F.Cu") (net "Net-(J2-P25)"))
 (segment (start 103 53.8) (end 102.6 54.2) (width 0.2) (layer "F.Cu") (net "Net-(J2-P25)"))
 (segment (start 97.685 81.115) (end 93.8 81.115) (width 0.2) (layer "F.Cu") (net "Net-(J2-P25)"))
 (segment (start 103.4 53.8) (end 103 53.8) (width 0.2) (layer "F.Cu") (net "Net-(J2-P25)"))
 (via (at 103.4 53.8) (size 0.6) (drill 0.3) (layers "F.Cu" "B.Cu") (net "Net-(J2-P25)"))
 (segment (start 106.385 54.785) (end 109.8 54.785) (width 0.2) (layer "B.Cu") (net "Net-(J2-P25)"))
 (segment (start 103.4 53.8) (end 105.4 53.8) (width 0.2) (layer "B.Cu") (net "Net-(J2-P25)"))
 (segment (start 105.4 53.8) (end 106.385 54.785) (width 0.2) (layer "B.Cu") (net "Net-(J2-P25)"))
 (segment (start 96.435 70.035) (end 97.6 71.2) (width 0.2) (layer "F.Cu") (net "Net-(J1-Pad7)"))
 (segment (start 93.8 70.035) (end 96.435 70.035) (width 0.2) (layer "F.Cu") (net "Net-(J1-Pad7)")))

